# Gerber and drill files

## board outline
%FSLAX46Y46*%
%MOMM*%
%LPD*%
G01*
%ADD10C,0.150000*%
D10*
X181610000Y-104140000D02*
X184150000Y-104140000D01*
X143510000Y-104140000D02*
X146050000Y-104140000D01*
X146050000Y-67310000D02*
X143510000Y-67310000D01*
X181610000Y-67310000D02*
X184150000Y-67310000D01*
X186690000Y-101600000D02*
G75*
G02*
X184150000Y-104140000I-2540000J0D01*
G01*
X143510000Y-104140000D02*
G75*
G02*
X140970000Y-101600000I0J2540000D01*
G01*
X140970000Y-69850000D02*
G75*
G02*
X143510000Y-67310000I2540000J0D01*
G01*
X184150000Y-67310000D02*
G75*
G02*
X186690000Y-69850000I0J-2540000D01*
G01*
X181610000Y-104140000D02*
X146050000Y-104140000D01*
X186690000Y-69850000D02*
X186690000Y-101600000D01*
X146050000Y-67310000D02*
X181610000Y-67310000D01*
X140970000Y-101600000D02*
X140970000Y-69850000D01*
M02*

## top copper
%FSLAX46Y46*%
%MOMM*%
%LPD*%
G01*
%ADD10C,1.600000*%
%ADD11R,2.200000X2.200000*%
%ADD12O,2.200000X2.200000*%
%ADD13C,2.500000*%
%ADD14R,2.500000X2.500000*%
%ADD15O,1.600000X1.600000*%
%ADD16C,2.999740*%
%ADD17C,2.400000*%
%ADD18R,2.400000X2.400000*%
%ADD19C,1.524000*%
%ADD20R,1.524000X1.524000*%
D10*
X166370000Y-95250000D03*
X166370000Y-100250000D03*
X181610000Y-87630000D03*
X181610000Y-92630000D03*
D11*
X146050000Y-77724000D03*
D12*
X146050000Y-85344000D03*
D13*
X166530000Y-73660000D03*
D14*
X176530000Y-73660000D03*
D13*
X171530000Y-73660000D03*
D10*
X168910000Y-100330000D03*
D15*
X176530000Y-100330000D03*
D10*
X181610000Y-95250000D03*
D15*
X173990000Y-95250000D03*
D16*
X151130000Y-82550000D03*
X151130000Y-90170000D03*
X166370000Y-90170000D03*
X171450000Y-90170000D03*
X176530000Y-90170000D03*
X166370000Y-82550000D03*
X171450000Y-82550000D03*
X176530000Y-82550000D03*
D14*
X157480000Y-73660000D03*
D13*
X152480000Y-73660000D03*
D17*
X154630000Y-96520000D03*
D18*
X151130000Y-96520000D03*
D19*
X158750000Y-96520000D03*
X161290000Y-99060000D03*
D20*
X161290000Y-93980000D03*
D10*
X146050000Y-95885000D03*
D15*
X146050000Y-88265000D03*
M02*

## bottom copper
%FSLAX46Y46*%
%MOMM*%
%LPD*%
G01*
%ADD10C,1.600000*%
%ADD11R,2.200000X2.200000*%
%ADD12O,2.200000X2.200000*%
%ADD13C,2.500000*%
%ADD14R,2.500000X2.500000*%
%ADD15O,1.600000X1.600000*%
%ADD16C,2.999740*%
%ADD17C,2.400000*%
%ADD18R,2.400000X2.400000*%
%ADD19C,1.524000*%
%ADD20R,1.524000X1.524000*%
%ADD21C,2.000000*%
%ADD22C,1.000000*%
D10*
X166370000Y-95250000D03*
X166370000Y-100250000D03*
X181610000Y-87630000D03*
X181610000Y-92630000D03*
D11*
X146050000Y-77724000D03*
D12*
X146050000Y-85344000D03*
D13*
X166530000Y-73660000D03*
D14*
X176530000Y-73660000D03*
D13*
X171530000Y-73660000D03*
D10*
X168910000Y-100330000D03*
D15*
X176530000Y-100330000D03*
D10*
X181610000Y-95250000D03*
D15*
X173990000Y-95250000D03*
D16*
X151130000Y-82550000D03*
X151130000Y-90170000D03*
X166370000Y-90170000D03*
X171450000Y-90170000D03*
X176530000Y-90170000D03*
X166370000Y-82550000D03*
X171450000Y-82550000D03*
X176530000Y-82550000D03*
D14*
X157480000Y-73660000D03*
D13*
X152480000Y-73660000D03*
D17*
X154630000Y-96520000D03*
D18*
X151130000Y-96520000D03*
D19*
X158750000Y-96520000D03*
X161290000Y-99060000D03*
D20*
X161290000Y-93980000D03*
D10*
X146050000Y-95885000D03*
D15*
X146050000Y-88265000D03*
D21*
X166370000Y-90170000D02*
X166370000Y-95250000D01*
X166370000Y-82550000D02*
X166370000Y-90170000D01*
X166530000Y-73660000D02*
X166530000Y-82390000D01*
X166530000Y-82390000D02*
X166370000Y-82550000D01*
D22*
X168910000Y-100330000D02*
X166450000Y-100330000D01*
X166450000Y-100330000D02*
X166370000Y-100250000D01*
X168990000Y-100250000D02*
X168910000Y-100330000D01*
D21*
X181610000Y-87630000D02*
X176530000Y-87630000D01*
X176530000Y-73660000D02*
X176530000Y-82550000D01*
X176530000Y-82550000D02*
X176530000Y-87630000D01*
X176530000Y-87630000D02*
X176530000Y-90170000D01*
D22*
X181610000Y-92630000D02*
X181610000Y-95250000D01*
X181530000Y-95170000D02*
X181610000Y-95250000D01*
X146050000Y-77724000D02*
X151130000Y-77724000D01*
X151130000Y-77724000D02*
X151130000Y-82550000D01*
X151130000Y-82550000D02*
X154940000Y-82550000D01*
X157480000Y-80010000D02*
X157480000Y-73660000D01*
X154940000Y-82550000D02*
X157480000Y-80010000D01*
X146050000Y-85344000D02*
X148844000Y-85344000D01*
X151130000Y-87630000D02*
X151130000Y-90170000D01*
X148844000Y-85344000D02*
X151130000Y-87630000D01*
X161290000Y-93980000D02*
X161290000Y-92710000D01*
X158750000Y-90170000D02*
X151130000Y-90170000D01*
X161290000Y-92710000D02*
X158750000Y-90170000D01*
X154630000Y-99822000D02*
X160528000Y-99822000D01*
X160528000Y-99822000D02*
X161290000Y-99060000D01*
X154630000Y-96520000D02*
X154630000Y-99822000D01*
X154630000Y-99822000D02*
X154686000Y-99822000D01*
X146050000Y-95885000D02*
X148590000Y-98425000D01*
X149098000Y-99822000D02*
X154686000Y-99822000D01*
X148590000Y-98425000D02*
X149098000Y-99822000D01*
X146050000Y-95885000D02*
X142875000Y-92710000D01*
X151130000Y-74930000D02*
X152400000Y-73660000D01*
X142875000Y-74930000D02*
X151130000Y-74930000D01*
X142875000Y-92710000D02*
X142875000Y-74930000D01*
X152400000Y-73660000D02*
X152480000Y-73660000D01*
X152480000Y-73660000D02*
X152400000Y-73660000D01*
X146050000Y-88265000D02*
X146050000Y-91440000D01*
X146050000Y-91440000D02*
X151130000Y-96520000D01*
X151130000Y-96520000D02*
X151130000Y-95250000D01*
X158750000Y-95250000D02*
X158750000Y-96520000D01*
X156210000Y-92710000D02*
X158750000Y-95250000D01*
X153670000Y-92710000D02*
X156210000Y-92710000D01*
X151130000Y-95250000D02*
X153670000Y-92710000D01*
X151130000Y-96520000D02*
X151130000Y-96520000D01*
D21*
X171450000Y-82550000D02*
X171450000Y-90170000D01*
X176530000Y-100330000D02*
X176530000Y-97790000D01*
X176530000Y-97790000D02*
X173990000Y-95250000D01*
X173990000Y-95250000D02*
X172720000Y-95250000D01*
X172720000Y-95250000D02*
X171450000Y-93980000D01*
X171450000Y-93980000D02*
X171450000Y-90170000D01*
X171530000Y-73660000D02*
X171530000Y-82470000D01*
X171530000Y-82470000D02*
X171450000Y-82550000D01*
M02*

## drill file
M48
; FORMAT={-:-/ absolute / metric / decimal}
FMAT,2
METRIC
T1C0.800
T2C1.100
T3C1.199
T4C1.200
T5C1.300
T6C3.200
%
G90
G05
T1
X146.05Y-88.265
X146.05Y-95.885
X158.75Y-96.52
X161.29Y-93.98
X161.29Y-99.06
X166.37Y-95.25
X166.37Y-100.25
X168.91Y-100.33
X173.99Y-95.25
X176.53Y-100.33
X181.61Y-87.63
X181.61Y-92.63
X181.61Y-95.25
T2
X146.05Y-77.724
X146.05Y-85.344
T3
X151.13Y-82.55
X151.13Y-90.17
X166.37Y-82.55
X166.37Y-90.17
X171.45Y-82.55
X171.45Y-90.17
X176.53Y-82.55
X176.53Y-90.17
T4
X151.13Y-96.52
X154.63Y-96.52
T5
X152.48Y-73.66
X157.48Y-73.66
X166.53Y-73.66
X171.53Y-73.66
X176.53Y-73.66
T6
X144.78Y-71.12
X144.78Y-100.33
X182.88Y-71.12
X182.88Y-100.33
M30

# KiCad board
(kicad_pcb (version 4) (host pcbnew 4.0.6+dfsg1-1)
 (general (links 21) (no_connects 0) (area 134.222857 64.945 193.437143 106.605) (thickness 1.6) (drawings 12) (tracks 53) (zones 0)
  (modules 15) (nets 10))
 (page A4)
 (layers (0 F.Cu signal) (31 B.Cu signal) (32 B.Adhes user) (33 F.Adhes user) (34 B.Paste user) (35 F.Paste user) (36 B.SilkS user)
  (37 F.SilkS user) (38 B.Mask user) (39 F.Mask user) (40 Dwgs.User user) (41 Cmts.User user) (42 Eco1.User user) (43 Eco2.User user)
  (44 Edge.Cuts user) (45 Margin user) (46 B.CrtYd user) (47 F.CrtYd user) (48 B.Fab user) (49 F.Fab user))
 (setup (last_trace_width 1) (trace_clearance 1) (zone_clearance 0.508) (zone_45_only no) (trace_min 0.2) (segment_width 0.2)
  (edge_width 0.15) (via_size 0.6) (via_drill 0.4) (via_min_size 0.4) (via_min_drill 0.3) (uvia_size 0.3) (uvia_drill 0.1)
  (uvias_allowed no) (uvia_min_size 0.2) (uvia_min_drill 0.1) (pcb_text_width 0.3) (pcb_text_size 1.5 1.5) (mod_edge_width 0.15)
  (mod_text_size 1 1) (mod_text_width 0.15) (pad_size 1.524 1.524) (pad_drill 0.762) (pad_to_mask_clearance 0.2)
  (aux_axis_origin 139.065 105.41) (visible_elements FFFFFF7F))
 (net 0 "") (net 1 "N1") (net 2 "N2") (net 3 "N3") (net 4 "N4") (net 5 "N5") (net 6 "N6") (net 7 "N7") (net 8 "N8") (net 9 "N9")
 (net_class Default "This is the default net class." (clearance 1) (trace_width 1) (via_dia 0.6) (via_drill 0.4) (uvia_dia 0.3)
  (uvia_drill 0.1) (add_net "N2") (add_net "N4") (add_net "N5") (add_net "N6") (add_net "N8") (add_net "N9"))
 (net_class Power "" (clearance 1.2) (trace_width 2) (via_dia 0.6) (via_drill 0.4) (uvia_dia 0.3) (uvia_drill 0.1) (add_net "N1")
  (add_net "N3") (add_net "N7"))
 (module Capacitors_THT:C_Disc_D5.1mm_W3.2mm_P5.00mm (layer F.Cu) (at 166.37 95.25 270)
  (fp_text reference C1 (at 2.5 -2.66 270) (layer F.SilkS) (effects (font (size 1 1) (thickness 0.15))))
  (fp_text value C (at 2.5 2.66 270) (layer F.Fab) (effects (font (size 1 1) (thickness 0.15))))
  (pad 1 thru_hole circle (at 0 0 270) (size 1.6 1.6) (drill 0.8) (layers *.Cu *.Mask) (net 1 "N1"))
  (pad 2 thru_hole circle (at 5 0 270) (size 1.6 1.6) (drill 0.8) (layers *.Cu *.Mask) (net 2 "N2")))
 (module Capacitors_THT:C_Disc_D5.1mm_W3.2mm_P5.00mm (layer F.Cu) (at 181.61 87.63 270)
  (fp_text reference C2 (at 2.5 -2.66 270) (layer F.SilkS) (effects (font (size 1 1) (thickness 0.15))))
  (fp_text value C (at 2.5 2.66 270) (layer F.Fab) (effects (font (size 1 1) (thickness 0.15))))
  (pad 1 thru_hole circle (at 0 0 270) (size 1.6 1.6) (drill 0.8) (layers *.Cu *.Mask) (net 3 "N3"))
  (pad 2 thru_hole circle (at 5 0 270) (size 1.6 1.6) (drill 0.8) (layers *.Cu *.Mask) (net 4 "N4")))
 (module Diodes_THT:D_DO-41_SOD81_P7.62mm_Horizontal (layer F.Cu) (at 146.05 77.724 270)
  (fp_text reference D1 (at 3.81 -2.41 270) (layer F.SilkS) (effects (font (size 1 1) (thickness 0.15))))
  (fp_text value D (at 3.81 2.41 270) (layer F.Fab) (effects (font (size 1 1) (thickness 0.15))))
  (pad 1 thru_hole rect (at 0 0 270) (size 2.2 2.2) (drill 1.1) (layers *.Cu *.Mask) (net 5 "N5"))
  (pad 2 thru_hole oval (at 7.62 0 270) (size 2.2 2.2) (drill 1.1) (layers *.Cu *.Mask) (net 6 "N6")))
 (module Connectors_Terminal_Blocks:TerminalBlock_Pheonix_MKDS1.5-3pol (layer F.Cu) (at 176.53 73.66 180)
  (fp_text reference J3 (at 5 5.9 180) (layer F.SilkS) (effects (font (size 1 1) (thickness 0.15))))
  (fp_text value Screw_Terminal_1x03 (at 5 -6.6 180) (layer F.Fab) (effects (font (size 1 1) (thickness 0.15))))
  (pad 3 thru_hole circle (at 10 0 180) (size 2.5 2.5) (drill 1.3) (layers *.Cu *.Mask) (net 1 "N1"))
  (pad 1 thru_hole rect (at 0 0 180) (size 2.5 2.5) (drill 1.3) (layers *.Cu *.Mask) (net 3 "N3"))
  (pad 2 thru_hole circle (at 5 0 180) (size 2.5 2.5) (drill 1.3) (layers *.Cu *.Mask) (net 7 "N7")))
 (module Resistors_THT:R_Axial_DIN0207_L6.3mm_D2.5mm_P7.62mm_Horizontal (layer F.Cu) (at 168.91 100.33)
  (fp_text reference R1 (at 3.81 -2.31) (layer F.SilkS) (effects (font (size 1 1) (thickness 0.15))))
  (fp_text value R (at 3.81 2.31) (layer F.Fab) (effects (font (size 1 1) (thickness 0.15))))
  (pad 1 thru_hole circle (at 0 0) (size 1.6 1.6) (drill 0.8) (layers *.Cu *.Mask) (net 2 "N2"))
  (pad 2 thru_hole oval (at 7.62 0) (size 1.6 1.6) (drill 0.8) (layers *.Cu *.Mask) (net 7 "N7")))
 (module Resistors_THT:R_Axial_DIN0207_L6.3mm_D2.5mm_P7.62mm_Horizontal (layer F.Cu) (at 181.61 95.25 180)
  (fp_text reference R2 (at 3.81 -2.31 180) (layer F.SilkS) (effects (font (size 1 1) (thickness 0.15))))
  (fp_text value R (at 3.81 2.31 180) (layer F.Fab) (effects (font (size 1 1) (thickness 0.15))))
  (pad 1 thru_hole circle (at 0 0 180) (size 1.6 1.6) (drill 0.8) (layers *.Cu *.Mask) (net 4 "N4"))
  (pad 2 thru_hole oval (at 7.62 0 180) (size 1.6 1.6) (drill 0.8) (layers *.Cu *.Mask) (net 7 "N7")))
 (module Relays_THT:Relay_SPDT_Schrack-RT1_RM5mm (layer F.Cu) (at 151.13 90.17)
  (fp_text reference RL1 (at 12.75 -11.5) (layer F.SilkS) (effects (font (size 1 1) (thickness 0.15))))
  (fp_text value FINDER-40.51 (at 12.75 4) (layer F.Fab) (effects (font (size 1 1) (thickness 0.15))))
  (pad A1 thru_hole circle (at 0 -7.62) (size 2.99974 2.99974) (drill 1.19888) (layers *.Cu *.Mask) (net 5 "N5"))
  (pad A2 thru_hole circle (at 0 0) (size 2.99974 2.99974) (drill 1.19888) (layers *.Cu *.Mask) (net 6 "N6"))
  (pad 12 thru_hole circle (at 15.24 0) (size 2.99974 2.99974) (drill 1.19888) (layers *.Cu *.Mask) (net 1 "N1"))
  (pad 11 thru_hole circle (at 20.32 0) (size 2.99974 2.99974) (drill 1.19888) (layers *.Cu *.Mask) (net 7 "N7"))
  (pad 14 thru_hole circle (at 25.4 0) (size 2.99974 2.99974) (drill 1.19888) (layers *.Cu *.Mask) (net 3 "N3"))
  (pad 12 thru_hole circle (at 15.24 -7.62) (size 2.99974 2.99974) (drill 1.19888) (layers *.Cu *.Mask) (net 1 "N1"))
  (pad 11 thru_hole circle (at 20.32 -7.62) (size 2.99974 2.99974) (drill 1.19888) (layers *.Cu *.Mask) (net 7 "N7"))
  (pad 14 thru_hole circle (at 25.4 -7.62) (size 2.99974 2.99974) (drill 1.19888) (layers *.Cu *.Mask) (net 3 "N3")))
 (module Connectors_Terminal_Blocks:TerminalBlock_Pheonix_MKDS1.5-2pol (layer F.Cu) (at 157.48 73.66 180)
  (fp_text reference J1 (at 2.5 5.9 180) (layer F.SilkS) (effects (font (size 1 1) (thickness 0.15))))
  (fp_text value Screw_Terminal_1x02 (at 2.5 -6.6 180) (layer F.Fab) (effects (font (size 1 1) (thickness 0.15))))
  (pad 1 thru_hole rect (at 0 0 180) (size 2.5 2.5) (drill 1.3) (layers *.Cu *.Mask) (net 5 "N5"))
  (pad 2 thru_hole circle (at 5 0 180) (size 2.5 2.5) (drill 1.3) (layers *.Cu *.Mask) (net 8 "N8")))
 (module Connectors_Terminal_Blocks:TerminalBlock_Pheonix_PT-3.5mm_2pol (layer F.Cu) (at 151.13 96.52)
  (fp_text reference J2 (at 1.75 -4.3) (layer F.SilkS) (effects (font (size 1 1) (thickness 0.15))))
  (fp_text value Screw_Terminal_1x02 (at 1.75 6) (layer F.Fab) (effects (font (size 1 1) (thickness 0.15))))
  (pad 2 thru_hole circle (at 3.5 0) (size 2.4 2.4) (drill 1.2) (layers *.Cu *.Mask) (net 8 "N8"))
  (pad 1 thru_hole rect (at 0 0) (size 2.4 2.4) (drill 1.2) (layers *.Cu *.Mask) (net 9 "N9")))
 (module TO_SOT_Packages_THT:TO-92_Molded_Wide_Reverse (layer F.Cu) (at 161.29 93.98 270)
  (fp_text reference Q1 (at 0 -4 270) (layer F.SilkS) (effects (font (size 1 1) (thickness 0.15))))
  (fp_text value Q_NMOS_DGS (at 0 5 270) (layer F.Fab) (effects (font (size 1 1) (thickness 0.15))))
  (pad 2 thru_hole circle (at 2.54 2.54) (size 1.524 1.524) (drill 0.8) (layers *.Cu *.Mask) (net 9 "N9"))
  (pad 3 thru_hole circle (at 5.08 0) (size 1.524 1.524) (drill 0.8) (layers *.Cu *.Mask) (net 8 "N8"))
  (pad 1 thru_hole rect (at 0 0) (size 1.524 1.524) (drill 0.8) (layers *.Cu *.Mask) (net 6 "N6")))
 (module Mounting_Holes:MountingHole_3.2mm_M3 (layer F.Cu) (at 144.78 71.12)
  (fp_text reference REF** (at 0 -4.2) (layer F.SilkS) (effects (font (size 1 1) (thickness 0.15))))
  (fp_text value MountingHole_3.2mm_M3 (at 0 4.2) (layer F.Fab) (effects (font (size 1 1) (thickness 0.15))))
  (pad 1 np_thru_hole circle (at 0 0) (size 3.2 3.2) (drill 3.2) (layers *.Cu *.Mask)))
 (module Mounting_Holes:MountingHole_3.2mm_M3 (layer F.Cu) (at 182.88 71.12)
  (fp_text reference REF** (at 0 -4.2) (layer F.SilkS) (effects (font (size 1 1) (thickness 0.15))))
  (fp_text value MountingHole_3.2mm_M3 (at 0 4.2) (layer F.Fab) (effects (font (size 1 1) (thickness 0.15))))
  (pad 1 np_thru_hole circle (at 0 0) (size 3.2 3.2) (drill 3.2) (layers *.Cu *.Mask)))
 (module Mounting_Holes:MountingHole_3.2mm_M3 (layer F.Cu) (at 182.88 100.33)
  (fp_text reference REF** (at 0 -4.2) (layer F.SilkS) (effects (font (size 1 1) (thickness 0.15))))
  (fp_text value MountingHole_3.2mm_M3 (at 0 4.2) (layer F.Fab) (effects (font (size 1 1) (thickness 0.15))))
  (pad 1 np_thru_hole circle (at 0 0) (size 3.2 3.2) (drill 3.2) (layers *.Cu *.Mask)))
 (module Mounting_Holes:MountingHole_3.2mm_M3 (layer F.Cu) (at 144.78 100.33)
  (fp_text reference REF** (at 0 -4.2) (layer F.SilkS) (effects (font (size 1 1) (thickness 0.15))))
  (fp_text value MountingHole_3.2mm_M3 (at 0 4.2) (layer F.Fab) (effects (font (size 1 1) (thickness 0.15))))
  (pad 1 np_thru_hole circle (at 0 0) (size 3.2 3.2) (drill 3.2) (layers *.Cu *.Mask)))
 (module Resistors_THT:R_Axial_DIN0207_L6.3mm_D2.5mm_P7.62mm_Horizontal (layer F.Cu) (at 146.05 95.885 90)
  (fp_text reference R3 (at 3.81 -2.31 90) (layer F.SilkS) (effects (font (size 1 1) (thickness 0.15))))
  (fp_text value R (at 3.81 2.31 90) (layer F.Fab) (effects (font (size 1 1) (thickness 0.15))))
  (pad 1 thru_hole circle (at 0 0 90) (size 1.6 1.6) (drill 0.8) (layers *.Cu *.Mask) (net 8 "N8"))
  (pad 2 thru_hole oval (at 7.62 0 90) (size 1.6 1.6) (drill 0.8) (layers *.Cu *.Mask) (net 9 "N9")))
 (gr_line (start 181.61 104.14) (end 184.15 104.14) (angle 90) (layer Edge.Cuts) (width 0.15))
 (gr_line (start 143.51 104.14) (end 146.05 104.14) (angle 90) (layer Edge.Cuts) (width 0.15))
 (gr_line (start 146.05 67.31) (end 143.51 67.31) (angle 90) (layer Edge.Cuts) (width 0.15))
 (gr_line (start 181.61 67.31) (end 184.15 67.31) (angle 90) (layer Edge.Cuts) (width 0.15))
 (gr_arc (start 184.15 101.6) (end 186.69 101.6) (angle 90) (layer Edge.Cuts) (width 0.15))
 (gr_arc (start 143.51 101.6) (end 143.51 104.14) (angle 90) (layer Edge.Cuts) (width 0.15))
 (gr_arc (start 143.51 69.85) (end 140.97 69.85) (angle 90) (layer Edge.Cuts) (width 0.15))
 (gr_arc (start 184.15 69.85) (end 184.15 67.31) (angle 90) (layer Edge.Cuts) (width 0.15))
 (gr_line (start 181.61 104.14) (end 146.05 104.14) (angle 90) (layer Edge.Cuts) (width 0.15))
 (gr_line (start 186.69 69.85) (end 186.69 101.6) (angle 90) (layer Edge.Cuts) (width 0.15))
 (gr_line (start 146.05 67.31) (end 181.61 67.31) (angle 90) (layer Edge.Cuts) (width 0.15))
 (gr_line (start 140.97 101.6) (end 140.97 69.85) (angle 90) (layer Edge.Cuts) (width 0.15))
 (segment (start 166.37 90.17) (end 166.37 95.25) (width 2) (layer B.Cu) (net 1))
 (segment (start 166.37 82.55) (end 166.37 90.17) (width 2) (layer B.Cu) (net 1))
 (segment (start 166.53 73.66) (end 166.53 82.39) (width 2) (layer B.Cu) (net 1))
 (segment (start 166.53 82.39) (end 166.37 82.55) (width 2) (layer B.Cu) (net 1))
 (segment (start 168.91 100.33) (end 166.45 100.33) (width 1) (layer B.Cu) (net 2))
 (segment (start 166.45 100.33) (end 166.37 100.25) (width 1) (layer B.Cu) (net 2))
 (segment (start 168.99 100.25) (end 168.91 100.33) (width 1) (layer B.Cu) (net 2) (status 30))
 (segment (start 181.61 87.63) (end 176.53 87.63) (width 2) (layer B.Cu) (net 3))
 (segment (start 176.53 73.66) (end 176.53 82.55) (width 2) (layer B.Cu) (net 3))
 (segment (start 176.53 82.55) (end 176.53 87.63) (width 2) (layer B.Cu) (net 3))
 (segment (start 176.53 87.63) (end 176.53 90.17) (width 2) (layer B.Cu) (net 3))
 (segment (start 181.61 92.63) (end 181.61 95.25) (width 1) (layer B.Cu) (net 4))
 (segment (start 181.53 95.17) (end 181.61 95.25) (width 1) (layer B.Cu) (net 4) (status 30))
 (segment (start 146.05 77.724) (end 151.13 77.724) (width 1) (layer B.Cu) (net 5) (status 400010))
 (segment (start 151.13 77.724) (end 151.13 82.55) (width 1) (layer B.Cu) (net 5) (status 800000))
 (segment (start 151.13 82.55) (end 154.94 82.55) (width 1) (layer B.Cu) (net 5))
 (segment (start 157.48 80.01) (end 157.48 73.66) (width 1) (layer B.Cu) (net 5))
 (segment (start 154.94 82.55) (end 157.48 80.01) (width 1) (layer B.Cu) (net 5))
 (segment (start 146.05 85.344) (end 148.844 85.344) (width 1) (layer B.Cu) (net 6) (status 400010))
 (segment (start 151.13 87.63) (end 151.13 90.17) (width 1) (layer B.Cu) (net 6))
 (segment (start 148.844 85.344) (end 151.13 87.63) (width 1) (layer B.Cu) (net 6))
 (segment (start 161.29 93.98) (end 161.29 92.71) (width 1) (layer B.Cu) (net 6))
 (segment (start 158.75 90.17) (end 151.13 90.17) (width 1) (layer B.Cu) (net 6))
 (segment (start 161.29 92.71) (end 158.75 90.17) (width 1) (layer B.Cu) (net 6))
 (segment (start 154.63 99.822) (end 160.528 99.822) (width 1) (layer B.Cu) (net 8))
 (segment (start 160.528 99.822) (end 161.29 99.06) (width 1) (layer B.Cu) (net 8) (status 800000))
 (segment (start 154.63 96.52) (end 154.63 99.822) (width 1) (layer B.Cu) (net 8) (status 400000))
 (segment (start 154.63 99.822) (end 154.686 99.822) (width 1) (layer B.Cu) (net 8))
 (segment (start 146.05 95.885) (end 148.59 98.425) (width 1) (layer B.Cu) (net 8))
 (segment (start 149.098 99.822) (end 154.686 99.822) (width 1) (layer B.Cu) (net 8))
 (segment (start 148.59 98.425) (end 149.098 99.822) (width 1) (layer B.Cu) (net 8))
 (segment (start 146.05 95.885) (end 142.875 92.71) (width 1) (layer B.Cu) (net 8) (status 10))
 (segment (start 151.13 74.93) (end 152.4 73.66) (width 1) (layer B.Cu) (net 8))
 (segment (start 142.875 74.93) (end 151.13 74.93) (width 1) (layer B.Cu) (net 8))
 (segment (start 142.875 92.71) (end 142.875 74.93) (width 1) (layer B.Cu) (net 8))
 (segment (start 152.4 73.66) (end 152.48 73.66) (width 1) (layer B.Cu) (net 8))
 (segment (start 152.48 73.66) (end 152.4 73.66) (width 1) (layer B.Cu) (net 8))
 (segment (start 146.05 88.265) (end 146.05 91.44) (width 1) (layer B.Cu) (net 9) (status 10))
 (segment (start 146.05 91.44) (end 151.13 96.52) (width 1) (layer B.Cu) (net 9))
 (segment (start 151.13 96.52) (end 151.13 95.25) (width 1) (layer B.Cu) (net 9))
 (segment (start 158.75 95.25) (end 158.75 96.52) (width 1) (layer B.Cu) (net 9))
 (segment (start 156.21 92.71) (end 158.75 95.25) (width 1) (layer B.Cu) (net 9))
 (segment (start 153.67 92.71) (end 156.21 92.71) (width 1) (layer B.Cu) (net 9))
 (segment (start 151.13 95.25) (end 153.67 92.71) (width 1) (layer B.Cu) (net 9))
 (segment (start 151.13 96.52) (end 151.13 96.52) (width 1) (layer B.Cu) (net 9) (status 30))
 (segment (start 171.45 82.55) (end 171.45 90.17) (width 2) (layer B.Cu) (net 7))
 (segment (start 176.53 100.33) (end 176.53 97.79) (width 2) (layer B.Cu) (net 7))
 (segment (start 176.53 97.79) (end 173.99 95.25) (width 2) (layer B.Cu) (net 7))
 (segment (start 173.99 95.25) (end 172.72 95.25) (width 2) (layer B.Cu) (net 7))
 (segment (start 172.72 95.25) (end 171.45 93.98) (width 2) (layer B.Cu) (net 7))
 (segment (start 171.45 93.98) (end 171.45 90.17) (width 2) (layer B.Cu) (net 7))
 (segment (start 171.53 73.66) (end 171.53 82.47) (width 2) (layer B.Cu) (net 7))
 (segment (start 171.53 82.47) (end 171.45 82.55) (width 2) (layer B.Cu) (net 7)))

